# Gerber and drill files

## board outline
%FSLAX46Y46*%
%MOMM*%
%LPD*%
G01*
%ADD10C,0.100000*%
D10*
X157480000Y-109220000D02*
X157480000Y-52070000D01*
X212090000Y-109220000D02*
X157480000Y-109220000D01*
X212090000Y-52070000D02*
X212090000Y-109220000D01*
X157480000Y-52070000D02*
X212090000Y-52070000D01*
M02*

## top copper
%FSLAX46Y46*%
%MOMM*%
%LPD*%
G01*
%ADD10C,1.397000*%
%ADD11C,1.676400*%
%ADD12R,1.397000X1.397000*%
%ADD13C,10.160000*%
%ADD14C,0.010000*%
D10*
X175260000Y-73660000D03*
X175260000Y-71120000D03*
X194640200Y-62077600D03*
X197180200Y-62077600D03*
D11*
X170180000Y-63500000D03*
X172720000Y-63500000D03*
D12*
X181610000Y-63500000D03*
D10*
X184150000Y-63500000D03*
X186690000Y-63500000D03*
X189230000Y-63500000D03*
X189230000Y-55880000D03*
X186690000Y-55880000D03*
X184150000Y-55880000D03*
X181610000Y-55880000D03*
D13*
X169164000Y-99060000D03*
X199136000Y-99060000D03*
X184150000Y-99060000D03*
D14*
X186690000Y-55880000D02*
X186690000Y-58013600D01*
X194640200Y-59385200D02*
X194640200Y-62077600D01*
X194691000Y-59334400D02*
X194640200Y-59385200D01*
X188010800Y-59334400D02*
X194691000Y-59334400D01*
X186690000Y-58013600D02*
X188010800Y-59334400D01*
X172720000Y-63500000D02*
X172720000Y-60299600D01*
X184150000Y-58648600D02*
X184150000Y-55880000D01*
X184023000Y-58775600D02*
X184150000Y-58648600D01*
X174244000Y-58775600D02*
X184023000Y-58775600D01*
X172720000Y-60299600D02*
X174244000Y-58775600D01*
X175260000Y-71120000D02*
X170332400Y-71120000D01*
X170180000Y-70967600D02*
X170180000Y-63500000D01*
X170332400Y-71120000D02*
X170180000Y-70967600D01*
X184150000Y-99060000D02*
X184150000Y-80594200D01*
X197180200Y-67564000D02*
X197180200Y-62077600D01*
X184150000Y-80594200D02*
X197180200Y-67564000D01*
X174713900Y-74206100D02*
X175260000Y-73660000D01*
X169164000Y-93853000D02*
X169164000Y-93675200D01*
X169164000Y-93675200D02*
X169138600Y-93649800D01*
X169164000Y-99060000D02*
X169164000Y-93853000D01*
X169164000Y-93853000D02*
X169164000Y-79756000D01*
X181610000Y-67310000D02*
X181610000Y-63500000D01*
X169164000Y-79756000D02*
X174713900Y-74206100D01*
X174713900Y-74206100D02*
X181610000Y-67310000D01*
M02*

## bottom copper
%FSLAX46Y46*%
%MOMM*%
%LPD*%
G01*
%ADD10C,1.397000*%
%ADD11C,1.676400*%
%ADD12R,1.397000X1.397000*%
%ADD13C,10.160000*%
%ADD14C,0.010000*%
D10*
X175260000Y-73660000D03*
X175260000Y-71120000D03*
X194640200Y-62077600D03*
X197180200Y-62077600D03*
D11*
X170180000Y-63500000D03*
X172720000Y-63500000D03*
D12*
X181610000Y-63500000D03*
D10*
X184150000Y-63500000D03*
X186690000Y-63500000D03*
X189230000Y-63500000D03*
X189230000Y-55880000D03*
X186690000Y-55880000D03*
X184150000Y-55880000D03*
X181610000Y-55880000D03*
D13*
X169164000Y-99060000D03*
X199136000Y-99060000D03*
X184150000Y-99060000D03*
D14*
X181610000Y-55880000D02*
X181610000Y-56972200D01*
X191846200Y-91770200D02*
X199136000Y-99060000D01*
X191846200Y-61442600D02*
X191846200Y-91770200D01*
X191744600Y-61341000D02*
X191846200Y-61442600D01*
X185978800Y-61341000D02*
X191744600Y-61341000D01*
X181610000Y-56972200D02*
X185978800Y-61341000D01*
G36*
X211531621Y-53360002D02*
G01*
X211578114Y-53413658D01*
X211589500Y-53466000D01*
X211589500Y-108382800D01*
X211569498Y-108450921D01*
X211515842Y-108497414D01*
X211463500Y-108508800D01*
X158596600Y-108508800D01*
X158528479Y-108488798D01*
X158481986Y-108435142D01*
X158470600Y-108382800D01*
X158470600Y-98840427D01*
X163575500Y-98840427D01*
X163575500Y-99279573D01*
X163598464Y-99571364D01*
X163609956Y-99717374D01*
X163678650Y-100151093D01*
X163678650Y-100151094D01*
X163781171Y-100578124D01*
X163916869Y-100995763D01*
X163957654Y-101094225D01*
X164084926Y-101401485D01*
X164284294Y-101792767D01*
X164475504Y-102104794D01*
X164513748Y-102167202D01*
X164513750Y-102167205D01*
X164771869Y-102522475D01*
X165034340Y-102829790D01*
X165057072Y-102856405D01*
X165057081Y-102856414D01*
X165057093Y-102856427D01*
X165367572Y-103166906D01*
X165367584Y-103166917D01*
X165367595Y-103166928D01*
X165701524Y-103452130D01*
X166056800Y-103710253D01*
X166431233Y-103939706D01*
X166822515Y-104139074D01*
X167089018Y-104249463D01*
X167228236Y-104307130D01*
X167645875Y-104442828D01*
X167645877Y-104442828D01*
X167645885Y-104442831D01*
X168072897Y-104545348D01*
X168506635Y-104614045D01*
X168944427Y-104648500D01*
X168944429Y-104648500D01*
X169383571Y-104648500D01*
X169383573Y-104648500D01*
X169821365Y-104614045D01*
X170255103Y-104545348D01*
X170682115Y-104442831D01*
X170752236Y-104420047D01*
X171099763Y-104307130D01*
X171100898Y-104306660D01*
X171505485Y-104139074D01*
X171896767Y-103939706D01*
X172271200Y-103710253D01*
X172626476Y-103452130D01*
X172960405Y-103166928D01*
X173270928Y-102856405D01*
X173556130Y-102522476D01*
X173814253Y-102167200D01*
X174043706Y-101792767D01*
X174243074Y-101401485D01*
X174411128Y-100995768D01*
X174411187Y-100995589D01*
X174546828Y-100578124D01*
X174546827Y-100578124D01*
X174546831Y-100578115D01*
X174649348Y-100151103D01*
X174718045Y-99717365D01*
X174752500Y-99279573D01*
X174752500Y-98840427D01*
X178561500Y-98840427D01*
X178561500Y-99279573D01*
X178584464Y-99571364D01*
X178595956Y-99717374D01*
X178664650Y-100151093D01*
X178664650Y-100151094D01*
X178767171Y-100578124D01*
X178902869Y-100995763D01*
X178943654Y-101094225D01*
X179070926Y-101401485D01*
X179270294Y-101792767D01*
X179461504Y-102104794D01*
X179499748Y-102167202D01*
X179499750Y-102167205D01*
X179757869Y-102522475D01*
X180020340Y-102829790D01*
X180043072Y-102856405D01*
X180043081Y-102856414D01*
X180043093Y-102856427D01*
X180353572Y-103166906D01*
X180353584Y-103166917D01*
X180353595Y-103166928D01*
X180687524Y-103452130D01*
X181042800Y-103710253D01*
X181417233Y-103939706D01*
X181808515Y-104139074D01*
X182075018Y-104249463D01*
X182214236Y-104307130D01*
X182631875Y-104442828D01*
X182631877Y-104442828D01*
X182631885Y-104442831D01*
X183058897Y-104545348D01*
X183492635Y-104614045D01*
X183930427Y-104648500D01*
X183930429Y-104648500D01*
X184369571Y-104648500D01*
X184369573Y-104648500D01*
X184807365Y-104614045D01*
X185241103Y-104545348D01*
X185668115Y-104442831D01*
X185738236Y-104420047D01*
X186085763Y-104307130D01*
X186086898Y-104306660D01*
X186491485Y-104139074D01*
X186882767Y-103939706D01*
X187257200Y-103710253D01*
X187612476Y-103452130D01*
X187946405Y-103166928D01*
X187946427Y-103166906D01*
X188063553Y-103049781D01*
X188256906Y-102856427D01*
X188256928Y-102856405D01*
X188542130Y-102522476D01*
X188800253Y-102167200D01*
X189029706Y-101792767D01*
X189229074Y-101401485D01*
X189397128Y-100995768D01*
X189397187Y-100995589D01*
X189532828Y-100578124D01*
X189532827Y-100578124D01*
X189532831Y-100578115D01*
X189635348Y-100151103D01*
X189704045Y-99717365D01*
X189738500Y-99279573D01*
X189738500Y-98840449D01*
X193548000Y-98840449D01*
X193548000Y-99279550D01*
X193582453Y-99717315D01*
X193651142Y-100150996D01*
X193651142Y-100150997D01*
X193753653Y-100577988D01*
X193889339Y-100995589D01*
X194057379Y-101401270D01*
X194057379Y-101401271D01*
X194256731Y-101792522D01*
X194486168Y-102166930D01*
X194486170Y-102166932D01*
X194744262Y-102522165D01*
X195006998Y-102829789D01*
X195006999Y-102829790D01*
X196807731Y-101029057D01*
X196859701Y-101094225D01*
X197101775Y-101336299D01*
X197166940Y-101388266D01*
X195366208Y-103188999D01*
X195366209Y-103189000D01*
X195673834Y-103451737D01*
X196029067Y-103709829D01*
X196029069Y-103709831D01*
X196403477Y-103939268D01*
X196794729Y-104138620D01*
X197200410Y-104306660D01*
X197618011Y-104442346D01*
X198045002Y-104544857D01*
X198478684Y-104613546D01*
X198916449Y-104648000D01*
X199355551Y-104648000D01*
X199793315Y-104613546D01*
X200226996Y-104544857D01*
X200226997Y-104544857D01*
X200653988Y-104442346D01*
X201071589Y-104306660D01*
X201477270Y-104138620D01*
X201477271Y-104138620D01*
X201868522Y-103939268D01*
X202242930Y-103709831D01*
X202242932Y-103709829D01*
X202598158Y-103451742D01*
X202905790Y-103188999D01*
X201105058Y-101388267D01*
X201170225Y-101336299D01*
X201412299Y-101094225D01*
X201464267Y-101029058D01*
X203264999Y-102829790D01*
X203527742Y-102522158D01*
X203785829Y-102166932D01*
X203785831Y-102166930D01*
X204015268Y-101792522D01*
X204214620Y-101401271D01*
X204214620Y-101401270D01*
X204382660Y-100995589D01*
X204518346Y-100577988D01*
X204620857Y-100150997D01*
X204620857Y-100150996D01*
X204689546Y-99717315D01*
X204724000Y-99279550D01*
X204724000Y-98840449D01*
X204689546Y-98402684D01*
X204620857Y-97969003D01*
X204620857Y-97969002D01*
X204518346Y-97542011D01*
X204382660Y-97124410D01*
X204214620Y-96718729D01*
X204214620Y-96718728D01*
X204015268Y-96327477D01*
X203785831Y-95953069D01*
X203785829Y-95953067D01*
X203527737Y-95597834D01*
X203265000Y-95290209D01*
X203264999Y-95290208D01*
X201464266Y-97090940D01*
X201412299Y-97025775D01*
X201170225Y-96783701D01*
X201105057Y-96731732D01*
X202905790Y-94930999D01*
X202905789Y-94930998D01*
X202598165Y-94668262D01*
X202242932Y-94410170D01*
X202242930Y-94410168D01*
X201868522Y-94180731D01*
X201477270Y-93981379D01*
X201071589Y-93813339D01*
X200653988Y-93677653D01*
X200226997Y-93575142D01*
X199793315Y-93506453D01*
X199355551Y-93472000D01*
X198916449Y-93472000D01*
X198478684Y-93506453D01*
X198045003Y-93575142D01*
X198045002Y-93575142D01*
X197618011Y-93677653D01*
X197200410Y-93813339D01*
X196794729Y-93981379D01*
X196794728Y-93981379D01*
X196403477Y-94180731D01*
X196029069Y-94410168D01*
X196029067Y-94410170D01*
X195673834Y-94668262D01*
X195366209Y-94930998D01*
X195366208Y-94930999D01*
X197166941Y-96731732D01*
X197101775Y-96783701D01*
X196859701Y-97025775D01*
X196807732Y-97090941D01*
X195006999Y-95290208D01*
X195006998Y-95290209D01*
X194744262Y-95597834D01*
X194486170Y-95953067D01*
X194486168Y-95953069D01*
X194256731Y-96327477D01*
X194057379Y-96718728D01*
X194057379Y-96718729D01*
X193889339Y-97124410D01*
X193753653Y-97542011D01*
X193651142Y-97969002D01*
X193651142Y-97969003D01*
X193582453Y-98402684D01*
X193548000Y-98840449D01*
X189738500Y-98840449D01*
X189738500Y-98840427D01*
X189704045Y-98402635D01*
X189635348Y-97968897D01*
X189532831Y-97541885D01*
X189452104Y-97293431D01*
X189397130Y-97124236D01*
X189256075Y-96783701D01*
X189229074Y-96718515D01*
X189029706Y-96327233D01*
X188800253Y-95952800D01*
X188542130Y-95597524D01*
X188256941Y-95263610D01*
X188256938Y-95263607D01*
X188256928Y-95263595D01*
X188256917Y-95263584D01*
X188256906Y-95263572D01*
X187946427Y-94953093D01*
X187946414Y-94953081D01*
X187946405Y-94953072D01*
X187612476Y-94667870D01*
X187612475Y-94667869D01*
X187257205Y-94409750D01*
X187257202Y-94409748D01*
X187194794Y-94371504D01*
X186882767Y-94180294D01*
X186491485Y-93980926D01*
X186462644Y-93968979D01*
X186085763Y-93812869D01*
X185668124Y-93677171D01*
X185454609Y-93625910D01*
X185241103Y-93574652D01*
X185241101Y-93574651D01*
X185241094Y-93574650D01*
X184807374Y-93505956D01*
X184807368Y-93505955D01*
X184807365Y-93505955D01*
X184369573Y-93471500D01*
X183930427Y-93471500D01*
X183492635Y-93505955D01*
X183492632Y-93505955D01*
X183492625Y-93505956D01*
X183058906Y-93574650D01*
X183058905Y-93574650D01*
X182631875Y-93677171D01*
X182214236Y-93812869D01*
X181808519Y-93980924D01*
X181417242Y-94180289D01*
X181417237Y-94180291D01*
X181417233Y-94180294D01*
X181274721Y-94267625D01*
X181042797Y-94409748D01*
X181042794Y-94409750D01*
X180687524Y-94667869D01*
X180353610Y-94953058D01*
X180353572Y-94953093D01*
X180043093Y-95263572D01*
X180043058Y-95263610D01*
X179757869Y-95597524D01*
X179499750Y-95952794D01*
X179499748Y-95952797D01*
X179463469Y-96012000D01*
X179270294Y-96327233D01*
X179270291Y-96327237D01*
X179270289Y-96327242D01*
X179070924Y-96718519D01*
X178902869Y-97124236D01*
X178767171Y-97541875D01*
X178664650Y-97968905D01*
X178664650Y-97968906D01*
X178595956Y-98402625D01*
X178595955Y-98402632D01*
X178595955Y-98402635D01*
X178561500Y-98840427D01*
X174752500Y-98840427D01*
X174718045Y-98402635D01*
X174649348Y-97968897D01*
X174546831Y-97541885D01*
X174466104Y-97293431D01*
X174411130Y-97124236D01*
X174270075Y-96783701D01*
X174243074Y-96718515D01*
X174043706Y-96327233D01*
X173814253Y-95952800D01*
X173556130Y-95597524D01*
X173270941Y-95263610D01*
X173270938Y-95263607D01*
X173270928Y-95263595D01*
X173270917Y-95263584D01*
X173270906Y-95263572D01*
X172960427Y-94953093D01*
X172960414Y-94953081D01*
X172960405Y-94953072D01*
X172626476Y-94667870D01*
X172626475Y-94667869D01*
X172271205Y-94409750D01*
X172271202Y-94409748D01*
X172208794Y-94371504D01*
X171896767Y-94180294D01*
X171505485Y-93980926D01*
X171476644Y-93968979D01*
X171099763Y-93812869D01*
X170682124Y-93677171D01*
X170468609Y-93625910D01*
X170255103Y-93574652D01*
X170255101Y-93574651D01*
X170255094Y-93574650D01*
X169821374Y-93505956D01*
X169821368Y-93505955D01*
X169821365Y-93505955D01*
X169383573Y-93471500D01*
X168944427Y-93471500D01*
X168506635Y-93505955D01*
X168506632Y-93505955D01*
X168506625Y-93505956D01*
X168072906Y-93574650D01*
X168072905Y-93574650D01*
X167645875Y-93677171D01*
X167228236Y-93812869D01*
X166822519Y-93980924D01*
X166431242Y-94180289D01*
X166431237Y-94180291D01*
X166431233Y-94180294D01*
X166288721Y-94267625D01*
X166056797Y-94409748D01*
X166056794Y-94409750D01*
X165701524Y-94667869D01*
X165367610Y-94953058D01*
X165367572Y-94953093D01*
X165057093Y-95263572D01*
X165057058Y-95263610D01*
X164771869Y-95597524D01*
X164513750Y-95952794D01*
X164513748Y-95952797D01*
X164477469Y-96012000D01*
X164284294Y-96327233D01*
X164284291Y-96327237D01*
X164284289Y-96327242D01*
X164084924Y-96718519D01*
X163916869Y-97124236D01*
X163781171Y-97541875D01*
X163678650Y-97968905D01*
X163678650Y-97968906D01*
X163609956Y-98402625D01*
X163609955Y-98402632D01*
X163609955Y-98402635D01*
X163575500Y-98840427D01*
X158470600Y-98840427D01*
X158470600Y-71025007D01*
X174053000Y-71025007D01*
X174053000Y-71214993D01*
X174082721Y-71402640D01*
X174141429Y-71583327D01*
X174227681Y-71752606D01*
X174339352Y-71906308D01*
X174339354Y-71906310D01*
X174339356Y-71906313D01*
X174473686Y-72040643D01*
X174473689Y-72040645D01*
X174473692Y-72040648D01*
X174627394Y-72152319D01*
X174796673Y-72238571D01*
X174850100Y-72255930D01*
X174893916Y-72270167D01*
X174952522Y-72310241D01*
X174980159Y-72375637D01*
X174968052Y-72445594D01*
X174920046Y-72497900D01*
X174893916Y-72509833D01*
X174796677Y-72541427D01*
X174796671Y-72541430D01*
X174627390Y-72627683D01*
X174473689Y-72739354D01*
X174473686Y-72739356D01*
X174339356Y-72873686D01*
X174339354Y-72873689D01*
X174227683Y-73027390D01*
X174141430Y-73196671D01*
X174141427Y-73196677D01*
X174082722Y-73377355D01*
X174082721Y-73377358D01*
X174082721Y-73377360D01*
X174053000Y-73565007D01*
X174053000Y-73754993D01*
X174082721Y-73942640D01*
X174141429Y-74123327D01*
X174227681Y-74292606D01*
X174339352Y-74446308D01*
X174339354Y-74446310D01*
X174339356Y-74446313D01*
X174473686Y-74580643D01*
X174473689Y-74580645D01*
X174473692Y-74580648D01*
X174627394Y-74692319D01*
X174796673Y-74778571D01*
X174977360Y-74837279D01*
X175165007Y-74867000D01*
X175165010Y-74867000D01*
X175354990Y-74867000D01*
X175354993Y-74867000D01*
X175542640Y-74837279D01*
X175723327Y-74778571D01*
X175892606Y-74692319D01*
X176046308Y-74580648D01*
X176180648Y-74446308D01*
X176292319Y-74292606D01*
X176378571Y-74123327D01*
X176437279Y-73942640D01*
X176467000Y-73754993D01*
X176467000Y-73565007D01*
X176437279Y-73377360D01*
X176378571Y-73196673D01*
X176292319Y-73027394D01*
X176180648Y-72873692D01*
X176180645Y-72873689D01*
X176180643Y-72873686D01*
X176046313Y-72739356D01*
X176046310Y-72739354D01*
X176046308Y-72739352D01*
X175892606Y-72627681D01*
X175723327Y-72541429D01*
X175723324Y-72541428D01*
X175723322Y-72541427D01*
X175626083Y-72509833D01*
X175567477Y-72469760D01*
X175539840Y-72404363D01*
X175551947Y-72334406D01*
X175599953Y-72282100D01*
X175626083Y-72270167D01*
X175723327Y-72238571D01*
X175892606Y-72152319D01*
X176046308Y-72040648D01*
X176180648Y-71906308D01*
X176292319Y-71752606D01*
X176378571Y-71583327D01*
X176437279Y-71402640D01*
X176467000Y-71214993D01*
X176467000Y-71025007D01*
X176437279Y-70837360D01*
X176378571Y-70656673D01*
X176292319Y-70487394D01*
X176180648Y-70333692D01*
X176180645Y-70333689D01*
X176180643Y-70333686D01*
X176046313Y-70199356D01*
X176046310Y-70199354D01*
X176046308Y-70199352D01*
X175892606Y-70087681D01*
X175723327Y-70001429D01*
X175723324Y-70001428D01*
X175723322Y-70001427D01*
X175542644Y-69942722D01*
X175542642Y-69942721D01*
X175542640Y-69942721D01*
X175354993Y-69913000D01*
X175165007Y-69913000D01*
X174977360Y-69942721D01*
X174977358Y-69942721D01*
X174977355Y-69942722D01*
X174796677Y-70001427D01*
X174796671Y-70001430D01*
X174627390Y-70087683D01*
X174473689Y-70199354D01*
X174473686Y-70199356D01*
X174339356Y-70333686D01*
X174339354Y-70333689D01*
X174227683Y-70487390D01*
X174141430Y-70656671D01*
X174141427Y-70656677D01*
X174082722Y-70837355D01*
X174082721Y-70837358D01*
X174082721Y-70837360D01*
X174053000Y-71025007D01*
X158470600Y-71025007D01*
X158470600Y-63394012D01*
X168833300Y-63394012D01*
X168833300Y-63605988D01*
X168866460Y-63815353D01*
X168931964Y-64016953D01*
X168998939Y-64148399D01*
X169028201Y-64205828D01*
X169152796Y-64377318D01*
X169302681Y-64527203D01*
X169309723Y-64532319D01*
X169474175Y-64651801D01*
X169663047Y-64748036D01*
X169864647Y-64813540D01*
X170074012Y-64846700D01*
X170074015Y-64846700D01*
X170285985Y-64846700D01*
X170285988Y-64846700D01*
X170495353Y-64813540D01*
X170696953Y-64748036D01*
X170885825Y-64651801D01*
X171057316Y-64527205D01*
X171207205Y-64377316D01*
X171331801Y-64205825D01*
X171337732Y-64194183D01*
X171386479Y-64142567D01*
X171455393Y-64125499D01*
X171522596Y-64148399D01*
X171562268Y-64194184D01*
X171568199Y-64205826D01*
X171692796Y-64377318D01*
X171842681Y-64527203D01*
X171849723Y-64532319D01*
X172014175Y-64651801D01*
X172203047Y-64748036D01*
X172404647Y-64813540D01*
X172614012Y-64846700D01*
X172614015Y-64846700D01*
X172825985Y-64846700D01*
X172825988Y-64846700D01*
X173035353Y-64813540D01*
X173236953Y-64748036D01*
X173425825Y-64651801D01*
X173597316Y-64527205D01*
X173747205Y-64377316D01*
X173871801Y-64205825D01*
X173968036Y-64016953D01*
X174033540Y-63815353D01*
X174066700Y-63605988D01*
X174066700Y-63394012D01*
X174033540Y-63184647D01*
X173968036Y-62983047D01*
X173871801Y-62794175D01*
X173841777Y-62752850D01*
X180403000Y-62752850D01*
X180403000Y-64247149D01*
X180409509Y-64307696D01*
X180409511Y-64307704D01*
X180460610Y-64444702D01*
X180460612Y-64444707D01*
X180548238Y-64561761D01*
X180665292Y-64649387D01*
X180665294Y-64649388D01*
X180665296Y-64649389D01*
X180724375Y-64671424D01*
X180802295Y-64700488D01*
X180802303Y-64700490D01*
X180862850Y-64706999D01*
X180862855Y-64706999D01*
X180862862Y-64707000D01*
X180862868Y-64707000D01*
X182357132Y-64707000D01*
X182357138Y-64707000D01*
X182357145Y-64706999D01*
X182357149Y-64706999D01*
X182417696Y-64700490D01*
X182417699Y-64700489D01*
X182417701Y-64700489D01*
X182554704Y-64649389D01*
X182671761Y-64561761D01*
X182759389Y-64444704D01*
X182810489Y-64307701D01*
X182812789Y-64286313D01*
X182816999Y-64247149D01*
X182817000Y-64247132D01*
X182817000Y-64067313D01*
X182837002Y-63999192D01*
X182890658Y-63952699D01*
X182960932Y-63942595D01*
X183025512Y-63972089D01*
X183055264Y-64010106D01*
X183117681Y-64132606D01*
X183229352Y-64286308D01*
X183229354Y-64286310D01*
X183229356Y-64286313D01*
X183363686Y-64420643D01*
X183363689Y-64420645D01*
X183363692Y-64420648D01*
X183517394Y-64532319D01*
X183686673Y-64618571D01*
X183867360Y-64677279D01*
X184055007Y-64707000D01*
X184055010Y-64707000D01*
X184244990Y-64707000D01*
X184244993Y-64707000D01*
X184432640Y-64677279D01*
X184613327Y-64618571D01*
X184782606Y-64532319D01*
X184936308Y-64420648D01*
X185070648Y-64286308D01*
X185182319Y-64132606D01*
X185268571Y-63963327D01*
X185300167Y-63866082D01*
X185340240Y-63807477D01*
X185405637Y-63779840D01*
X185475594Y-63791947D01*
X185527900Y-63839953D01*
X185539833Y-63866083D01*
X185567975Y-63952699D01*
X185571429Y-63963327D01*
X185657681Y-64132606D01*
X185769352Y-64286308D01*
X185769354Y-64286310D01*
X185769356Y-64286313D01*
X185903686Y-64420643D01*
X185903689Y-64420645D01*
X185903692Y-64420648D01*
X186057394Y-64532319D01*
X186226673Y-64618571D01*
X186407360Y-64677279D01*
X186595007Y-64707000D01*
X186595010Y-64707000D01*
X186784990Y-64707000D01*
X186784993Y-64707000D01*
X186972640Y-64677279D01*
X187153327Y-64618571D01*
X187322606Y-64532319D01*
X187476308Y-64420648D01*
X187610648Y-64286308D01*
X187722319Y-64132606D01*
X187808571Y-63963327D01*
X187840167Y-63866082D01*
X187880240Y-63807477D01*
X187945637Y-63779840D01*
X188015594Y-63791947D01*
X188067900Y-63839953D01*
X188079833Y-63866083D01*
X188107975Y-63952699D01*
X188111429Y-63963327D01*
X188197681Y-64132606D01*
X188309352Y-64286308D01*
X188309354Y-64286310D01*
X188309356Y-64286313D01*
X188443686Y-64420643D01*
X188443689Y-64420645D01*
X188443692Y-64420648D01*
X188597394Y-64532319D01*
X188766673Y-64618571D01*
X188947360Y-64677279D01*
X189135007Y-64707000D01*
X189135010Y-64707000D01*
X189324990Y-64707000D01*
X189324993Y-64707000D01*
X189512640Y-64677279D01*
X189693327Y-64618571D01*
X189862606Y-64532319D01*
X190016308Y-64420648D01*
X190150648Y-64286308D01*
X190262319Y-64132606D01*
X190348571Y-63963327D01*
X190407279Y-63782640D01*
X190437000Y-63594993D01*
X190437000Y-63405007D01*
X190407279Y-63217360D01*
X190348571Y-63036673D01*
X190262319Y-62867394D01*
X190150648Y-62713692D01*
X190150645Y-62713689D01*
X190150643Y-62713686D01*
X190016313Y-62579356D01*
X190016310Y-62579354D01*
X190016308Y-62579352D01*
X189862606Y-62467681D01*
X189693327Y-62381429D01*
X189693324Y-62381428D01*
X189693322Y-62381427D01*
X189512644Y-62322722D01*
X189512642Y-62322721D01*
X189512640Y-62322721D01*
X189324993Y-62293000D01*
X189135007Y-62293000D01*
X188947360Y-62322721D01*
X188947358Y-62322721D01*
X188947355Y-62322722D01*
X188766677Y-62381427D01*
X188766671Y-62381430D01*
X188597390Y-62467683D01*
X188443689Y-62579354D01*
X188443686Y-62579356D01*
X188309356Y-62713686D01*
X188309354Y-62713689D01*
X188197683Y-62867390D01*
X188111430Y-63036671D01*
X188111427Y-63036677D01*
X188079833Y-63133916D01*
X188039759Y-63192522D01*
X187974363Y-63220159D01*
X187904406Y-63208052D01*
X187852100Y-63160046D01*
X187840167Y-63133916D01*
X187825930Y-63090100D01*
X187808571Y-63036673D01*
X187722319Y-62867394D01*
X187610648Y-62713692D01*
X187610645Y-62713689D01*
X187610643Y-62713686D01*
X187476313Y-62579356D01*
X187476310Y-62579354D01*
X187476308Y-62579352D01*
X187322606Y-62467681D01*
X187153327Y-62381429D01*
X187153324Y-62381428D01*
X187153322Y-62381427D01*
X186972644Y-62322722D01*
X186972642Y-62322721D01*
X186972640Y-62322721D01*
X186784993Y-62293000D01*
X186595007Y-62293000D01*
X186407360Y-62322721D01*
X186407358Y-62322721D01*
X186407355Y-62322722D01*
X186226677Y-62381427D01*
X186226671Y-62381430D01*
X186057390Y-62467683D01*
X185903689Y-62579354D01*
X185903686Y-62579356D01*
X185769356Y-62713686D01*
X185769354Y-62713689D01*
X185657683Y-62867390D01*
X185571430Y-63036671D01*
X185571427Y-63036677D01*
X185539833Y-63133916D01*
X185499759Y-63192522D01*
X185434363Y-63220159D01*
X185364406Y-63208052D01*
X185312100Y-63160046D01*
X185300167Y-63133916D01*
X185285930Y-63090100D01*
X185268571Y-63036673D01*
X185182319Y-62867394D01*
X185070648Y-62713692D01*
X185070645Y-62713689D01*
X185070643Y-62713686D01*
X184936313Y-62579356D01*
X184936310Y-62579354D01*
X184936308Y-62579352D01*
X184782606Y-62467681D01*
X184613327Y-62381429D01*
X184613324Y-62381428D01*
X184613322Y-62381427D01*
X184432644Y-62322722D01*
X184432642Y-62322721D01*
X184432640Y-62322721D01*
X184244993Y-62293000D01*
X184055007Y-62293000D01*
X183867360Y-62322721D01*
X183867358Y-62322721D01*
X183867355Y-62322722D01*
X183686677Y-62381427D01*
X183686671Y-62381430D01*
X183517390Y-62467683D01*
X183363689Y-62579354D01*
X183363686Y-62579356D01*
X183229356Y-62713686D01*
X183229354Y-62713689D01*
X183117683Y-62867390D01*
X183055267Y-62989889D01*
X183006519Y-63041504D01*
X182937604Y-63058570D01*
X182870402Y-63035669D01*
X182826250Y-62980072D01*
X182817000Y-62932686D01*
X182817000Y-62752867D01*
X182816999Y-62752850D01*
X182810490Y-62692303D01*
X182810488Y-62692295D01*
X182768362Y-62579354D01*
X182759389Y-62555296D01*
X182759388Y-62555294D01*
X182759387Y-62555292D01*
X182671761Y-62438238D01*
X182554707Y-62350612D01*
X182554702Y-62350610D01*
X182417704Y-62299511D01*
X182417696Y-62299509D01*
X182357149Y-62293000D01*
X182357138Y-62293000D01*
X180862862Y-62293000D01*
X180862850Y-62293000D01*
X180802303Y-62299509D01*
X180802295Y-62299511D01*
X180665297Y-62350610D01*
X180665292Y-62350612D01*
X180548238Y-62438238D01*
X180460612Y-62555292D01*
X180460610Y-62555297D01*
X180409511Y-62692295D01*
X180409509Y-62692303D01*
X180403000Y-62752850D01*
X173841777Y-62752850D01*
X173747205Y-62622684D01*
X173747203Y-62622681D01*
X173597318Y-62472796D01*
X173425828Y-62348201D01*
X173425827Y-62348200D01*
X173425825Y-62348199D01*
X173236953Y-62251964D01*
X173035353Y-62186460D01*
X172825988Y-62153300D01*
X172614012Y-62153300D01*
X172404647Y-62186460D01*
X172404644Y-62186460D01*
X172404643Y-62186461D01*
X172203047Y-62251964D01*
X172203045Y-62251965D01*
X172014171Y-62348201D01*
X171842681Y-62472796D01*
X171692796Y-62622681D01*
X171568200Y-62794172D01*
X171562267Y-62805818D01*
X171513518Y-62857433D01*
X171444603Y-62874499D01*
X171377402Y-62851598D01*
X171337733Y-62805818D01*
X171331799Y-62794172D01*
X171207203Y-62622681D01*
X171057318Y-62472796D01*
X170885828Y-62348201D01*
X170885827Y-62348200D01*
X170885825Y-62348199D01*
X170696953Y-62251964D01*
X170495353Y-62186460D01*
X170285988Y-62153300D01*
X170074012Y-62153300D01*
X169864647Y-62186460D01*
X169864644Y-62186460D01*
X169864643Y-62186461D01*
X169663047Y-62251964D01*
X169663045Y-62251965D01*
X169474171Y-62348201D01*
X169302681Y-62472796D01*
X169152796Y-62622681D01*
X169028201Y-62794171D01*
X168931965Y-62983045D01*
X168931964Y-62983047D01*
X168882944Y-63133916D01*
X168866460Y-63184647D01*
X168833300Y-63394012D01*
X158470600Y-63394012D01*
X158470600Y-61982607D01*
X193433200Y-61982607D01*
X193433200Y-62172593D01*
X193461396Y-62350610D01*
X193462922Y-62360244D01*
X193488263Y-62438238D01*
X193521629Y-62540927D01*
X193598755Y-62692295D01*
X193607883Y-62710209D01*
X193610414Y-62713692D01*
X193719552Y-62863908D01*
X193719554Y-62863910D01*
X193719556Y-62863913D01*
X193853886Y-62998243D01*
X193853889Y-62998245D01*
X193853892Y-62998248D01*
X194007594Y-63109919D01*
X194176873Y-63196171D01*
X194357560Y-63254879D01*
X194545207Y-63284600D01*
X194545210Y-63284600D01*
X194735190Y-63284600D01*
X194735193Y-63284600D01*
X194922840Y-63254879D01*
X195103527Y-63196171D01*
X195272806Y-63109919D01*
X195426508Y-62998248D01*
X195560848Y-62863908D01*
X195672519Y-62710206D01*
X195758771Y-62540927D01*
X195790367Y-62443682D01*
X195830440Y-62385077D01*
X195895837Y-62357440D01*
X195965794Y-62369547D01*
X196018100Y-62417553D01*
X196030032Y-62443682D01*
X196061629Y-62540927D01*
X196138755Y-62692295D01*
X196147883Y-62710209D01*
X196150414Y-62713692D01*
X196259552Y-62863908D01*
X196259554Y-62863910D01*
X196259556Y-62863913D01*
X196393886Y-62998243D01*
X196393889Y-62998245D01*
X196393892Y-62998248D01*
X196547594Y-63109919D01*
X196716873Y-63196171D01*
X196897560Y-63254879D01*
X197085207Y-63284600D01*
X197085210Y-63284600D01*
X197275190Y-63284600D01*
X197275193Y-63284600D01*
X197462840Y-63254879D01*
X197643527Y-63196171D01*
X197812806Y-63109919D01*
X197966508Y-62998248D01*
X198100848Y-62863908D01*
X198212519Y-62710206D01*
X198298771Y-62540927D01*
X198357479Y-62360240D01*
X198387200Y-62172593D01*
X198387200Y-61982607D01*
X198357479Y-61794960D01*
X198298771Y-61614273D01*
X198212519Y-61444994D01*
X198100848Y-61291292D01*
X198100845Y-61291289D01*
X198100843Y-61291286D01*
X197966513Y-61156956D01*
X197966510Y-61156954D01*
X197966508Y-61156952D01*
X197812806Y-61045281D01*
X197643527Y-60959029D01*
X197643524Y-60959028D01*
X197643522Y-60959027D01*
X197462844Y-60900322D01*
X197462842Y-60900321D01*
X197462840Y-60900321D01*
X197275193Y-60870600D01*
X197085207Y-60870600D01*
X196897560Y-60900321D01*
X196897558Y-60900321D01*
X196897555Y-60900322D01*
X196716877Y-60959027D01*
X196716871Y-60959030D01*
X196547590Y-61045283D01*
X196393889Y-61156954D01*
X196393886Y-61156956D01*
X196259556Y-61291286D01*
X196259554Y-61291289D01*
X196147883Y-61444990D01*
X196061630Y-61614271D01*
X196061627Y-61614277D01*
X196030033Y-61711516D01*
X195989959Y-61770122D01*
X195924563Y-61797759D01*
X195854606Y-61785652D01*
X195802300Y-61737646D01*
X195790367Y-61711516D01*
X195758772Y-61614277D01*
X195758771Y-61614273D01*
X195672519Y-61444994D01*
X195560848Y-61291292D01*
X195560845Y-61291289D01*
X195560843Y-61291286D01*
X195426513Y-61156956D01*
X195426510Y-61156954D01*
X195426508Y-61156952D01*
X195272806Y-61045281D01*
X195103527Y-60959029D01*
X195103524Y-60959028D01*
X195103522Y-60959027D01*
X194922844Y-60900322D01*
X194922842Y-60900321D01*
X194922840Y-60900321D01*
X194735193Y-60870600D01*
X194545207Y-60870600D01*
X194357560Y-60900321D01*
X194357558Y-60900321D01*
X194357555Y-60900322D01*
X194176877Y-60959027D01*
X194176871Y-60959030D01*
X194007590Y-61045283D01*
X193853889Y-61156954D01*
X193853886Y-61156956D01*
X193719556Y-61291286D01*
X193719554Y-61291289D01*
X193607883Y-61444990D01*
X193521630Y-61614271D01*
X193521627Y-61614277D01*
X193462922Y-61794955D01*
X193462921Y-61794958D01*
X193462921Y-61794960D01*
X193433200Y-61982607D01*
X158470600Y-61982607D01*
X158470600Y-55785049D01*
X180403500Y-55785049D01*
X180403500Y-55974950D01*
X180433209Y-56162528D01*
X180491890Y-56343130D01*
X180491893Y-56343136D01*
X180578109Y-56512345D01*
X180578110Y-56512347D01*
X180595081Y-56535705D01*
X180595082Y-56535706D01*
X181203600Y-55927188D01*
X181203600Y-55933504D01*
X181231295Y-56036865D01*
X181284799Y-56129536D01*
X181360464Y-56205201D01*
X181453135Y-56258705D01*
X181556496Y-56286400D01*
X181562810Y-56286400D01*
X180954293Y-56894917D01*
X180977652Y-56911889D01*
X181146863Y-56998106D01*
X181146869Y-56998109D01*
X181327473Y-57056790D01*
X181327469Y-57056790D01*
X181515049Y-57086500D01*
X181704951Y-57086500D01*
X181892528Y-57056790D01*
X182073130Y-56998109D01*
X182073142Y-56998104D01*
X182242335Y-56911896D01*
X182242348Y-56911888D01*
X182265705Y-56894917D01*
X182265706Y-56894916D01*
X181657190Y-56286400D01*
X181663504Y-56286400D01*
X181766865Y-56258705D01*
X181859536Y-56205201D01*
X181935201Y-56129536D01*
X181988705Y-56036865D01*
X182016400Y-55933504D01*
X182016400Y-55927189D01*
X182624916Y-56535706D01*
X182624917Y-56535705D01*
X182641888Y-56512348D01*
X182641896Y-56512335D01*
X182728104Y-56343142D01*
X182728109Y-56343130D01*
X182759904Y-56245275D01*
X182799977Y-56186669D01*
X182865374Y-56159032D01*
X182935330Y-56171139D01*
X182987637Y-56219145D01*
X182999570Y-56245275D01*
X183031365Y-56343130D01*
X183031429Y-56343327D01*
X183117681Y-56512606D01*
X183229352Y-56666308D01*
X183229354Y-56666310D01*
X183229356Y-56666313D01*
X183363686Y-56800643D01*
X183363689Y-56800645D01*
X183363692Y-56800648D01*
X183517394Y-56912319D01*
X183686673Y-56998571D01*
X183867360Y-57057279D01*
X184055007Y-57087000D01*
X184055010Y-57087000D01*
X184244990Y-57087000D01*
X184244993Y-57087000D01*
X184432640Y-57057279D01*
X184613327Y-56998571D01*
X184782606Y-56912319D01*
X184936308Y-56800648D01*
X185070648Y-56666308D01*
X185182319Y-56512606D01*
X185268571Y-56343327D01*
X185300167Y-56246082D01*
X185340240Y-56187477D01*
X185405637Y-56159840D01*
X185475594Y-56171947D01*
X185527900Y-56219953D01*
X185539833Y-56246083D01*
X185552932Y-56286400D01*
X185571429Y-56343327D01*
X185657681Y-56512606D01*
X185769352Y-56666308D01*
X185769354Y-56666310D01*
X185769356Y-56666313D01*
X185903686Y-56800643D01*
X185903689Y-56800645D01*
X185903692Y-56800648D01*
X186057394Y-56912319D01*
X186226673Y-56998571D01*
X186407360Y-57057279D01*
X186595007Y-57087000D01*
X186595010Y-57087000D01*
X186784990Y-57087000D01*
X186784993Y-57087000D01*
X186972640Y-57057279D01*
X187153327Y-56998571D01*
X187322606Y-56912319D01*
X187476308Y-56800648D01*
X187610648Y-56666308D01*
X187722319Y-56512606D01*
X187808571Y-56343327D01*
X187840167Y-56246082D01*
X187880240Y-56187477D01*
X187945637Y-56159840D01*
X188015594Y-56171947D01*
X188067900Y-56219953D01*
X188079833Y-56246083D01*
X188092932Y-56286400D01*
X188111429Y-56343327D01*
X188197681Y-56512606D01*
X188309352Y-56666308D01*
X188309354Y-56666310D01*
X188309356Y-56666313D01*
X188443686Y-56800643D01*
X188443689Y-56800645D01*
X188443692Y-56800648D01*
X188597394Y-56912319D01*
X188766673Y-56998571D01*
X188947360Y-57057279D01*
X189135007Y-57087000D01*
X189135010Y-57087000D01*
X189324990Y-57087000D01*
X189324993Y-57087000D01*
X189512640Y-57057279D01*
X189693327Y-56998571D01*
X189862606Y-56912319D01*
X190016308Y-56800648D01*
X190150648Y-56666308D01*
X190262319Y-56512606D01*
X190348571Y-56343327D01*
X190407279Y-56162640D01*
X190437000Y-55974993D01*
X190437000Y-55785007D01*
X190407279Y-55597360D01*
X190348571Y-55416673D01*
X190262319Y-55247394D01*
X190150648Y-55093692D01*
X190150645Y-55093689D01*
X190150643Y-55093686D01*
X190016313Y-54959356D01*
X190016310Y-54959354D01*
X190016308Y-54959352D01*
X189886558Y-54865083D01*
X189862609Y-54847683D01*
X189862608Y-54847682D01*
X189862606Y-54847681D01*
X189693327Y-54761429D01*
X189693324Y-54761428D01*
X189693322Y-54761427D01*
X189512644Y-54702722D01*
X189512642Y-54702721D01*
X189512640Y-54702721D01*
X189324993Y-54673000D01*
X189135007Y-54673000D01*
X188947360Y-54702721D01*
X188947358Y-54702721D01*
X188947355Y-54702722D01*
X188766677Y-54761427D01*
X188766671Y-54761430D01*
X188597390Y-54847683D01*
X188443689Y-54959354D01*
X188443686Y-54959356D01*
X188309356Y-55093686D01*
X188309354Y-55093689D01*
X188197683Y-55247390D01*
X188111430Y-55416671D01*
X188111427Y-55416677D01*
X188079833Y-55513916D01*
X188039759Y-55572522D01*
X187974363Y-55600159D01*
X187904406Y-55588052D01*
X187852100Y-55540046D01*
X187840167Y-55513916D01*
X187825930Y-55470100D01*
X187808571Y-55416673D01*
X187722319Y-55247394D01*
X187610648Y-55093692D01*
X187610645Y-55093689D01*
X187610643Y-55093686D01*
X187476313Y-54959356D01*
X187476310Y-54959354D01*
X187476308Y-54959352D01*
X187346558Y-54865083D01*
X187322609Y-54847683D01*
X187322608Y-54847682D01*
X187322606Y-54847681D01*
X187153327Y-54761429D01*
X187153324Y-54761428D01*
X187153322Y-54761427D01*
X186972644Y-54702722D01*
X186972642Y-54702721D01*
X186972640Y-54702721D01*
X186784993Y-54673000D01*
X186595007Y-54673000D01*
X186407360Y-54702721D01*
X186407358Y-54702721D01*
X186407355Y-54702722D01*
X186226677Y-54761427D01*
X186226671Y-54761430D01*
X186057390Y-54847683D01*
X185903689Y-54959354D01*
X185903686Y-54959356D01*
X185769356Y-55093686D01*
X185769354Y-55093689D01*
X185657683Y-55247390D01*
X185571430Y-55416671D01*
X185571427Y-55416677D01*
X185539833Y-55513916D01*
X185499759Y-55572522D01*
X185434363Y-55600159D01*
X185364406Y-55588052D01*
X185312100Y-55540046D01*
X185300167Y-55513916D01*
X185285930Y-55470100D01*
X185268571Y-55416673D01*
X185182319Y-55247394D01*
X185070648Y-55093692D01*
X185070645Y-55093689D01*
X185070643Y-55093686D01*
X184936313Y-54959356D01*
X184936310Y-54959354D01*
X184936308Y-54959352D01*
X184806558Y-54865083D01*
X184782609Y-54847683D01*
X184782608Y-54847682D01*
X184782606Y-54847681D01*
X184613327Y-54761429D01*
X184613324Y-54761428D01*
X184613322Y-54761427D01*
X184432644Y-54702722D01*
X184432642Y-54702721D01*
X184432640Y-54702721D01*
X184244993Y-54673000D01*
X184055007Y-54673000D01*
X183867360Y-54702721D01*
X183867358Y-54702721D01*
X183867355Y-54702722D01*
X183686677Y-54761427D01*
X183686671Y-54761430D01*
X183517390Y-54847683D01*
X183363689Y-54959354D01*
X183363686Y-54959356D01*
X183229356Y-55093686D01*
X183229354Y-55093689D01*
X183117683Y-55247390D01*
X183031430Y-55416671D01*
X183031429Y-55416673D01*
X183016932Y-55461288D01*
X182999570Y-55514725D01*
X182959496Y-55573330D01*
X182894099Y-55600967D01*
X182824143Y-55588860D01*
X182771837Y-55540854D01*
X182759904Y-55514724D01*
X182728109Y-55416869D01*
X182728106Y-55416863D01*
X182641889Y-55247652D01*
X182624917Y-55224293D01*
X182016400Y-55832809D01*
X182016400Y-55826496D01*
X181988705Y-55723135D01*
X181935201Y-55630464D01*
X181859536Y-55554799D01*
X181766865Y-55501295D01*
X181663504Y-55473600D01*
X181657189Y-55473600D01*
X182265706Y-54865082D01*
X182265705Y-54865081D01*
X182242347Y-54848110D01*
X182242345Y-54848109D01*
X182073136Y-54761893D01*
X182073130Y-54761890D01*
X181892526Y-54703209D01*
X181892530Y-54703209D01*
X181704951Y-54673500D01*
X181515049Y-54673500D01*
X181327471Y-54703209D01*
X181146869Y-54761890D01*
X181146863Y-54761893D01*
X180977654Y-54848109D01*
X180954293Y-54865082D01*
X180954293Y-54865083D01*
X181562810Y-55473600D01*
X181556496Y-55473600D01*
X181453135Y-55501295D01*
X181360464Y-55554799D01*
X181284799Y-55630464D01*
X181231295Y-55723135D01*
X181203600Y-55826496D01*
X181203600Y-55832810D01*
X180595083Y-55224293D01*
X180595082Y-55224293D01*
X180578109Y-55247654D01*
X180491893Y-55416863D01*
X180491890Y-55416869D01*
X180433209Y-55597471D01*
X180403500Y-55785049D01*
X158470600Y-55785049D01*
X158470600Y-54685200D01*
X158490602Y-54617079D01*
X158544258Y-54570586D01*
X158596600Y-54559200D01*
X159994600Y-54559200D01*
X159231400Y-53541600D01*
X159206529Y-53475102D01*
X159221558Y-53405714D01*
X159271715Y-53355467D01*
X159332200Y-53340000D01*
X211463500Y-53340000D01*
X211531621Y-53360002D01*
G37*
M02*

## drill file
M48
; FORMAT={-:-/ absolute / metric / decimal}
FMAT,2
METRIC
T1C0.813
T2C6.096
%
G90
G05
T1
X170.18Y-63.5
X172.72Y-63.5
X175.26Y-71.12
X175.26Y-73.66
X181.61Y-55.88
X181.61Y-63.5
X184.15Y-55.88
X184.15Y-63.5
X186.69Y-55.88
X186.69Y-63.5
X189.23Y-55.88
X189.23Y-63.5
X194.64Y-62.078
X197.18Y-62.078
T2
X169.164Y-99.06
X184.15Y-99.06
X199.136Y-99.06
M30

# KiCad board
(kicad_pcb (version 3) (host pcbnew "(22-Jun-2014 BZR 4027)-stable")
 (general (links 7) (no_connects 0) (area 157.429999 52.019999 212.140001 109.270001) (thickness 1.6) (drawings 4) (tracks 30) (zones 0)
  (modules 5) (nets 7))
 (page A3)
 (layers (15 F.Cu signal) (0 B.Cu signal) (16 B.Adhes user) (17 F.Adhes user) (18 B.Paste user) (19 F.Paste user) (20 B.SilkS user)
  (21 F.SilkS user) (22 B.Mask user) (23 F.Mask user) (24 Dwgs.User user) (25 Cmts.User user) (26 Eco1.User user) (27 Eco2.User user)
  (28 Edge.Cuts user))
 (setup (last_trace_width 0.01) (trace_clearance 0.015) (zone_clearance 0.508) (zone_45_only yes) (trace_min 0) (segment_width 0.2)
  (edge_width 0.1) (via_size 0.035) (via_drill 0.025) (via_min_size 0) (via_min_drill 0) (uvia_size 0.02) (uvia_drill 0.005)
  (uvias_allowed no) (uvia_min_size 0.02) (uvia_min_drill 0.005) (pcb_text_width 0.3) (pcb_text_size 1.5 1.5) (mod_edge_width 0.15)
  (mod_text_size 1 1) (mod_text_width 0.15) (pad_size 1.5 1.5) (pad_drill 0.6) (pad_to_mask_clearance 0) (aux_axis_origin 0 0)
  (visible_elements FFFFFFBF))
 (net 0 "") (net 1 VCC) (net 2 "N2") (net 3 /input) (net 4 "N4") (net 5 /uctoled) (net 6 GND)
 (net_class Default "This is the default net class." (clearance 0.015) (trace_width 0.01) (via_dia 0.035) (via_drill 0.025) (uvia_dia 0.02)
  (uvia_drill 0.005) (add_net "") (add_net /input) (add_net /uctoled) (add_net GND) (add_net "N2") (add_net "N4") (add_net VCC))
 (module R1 (layer F.Cu) (at 175.26 72.39 90) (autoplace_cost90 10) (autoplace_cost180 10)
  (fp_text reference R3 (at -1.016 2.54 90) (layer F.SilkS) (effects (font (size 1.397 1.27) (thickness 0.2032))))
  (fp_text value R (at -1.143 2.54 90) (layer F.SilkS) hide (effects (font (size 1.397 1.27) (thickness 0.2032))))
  (pad 1 thru_hole circle (at -1.27 0 90) (size 1.397 1.397) (drill 0.8128) (layers *.Cu *.Mask F.SilkS) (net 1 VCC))
  (pad 2 thru_hole circle (at 1.27 0 90) (size 1.397 1.397) (drill 0.8128) (layers *.Cu *.Mask F.SilkS) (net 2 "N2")))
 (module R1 (layer F.Cu) (at 195.9102 62.0776) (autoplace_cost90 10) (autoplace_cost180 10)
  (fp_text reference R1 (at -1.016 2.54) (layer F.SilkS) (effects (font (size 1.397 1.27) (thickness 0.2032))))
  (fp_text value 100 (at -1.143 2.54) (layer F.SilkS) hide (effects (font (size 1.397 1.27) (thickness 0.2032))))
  (pad 1 thru_hole circle (at -1.27 0) (size 1.397 1.397) (drill 0.8128) (layers *.Cu *.Mask F.SilkS) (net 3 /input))
  (pad 2 thru_hole circle (at 1.27 0) (size 1.397 1.397) (drill 0.8128) (layers *.Cu *.Mask F.SilkS) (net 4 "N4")))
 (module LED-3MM (layer F.Cu) (at 171.45 63.5)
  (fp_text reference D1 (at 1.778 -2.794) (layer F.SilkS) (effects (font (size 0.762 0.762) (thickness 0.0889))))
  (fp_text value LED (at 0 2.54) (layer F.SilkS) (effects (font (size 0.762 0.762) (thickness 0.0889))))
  (pad 1 thru_hole circle (at -1.27 0) (size 1.6764 1.6764) (drill 0.8128) (layers *.Cu *.Mask F.SilkS) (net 2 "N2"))
  (pad 2 thru_hole circle (at 1.27 0) (size 1.6764 1.6764) (drill 0.8128) (layers *.Cu *.Mask F.SilkS) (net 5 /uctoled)))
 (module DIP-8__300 (layer F.Cu) (at 185.42 59.69)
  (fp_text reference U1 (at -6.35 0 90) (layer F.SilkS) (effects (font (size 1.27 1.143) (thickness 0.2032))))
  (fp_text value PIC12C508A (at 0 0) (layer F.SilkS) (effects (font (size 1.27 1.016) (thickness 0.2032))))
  (pad 1 thru_hole rect (at -3.81 3.81) (size 1.397 1.397) (drill 0.8128) (layers *.Cu *.Mask F.SilkS) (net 1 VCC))
  (pad 2 thru_hole circle (at -1.27 3.81) (size 1.397 1.397) (drill 0.8128) (layers *.Cu *.Mask F.SilkS))
  (pad 3 thru_hole circle (at 1.27 3.81) (size 1.397 1.397) (drill 0.8128) (layers *.Cu *.Mask F.SilkS))
  (pad 4 thru_hole circle (at 3.81 3.81) (size 1.397 1.397) (drill 0.8128) (layers *.Cu *.Mask F.SilkS))
  (pad 5 thru_hole circle (at 3.81 -3.81) (size 1.397 1.397) (drill 0.8128) (layers *.Cu *.Mask F.SilkS))
  (pad 6 thru_hole circle (at 1.27 -3.81) (size 1.397 1.397) (drill 0.8128) (layers *.Cu *.Mask F.SilkS) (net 3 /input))
  (pad 7 thru_hole circle (at -1.27 -3.81) (size 1.397 1.397) (drill 0.8128) (layers *.Cu *.Mask F.SilkS) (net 5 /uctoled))
  (pad 8 thru_hole circle (at -3.81 -3.81) (size 1.397 1.397) (drill 0.8128) (layers *.Cu *.Mask F.SilkS) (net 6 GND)))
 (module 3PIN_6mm (layer F.Cu) (at 184.15 99.06)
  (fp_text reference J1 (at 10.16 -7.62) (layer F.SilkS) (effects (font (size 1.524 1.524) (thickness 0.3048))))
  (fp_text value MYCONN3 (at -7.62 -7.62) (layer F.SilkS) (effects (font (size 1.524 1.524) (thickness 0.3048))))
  (pad 1 thru_hole circle (at -14.986 0) (size 10.16 10.16) (drill 6.096) (layers *.Cu *.Mask F.SilkS) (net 1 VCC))
  (pad 3 thru_hole circle (at 14.986 0) (size 10.16 10.16) (drill 6.096) (layers *.Cu *.Mask F.SilkS) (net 6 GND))
  (pad 2 thru_hole circle (at 0 0) (size 10.16 10.16) (drill 6.096) (layers *.Cu *.Mask F.SilkS) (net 4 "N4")))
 (gr_line (start 157.48 109.22) (end 157.48 52.07) (angle 90) (layer Edge.Cuts) (width 0.1))
 (gr_line (start 212.09 109.22) (end 157.48 109.22) (angle 90) (layer Edge.Cuts) (width 0.1))
 (gr_line (start 212.09 52.07) (end 212.09 109.22) (angle 90) (layer Edge.Cuts) (width 0.1))
 (gr_line (start 157.48 52.07) (end 212.09 52.07) (angle 90) (layer Edge.Cuts) (width 0.1))
 (segment (start 186.69 55.88) (end 186.69 58.0136) (width 0.01) (layer F.Cu) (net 3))
 (segment (start 194.6402 59.3852) (end 194.6402 62.0776) (width 0.01) (layer F.Cu) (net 3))
 (segment (start 194.691 59.3344) (end 194.6402 59.3852) (width 0.01) (layer F.Cu) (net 3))
 (segment (start 188.0108 59.3344) (end 194.691 59.3344) (width 0.01) (layer F.Cu) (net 3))
 (segment (start 186.69 58.0136) (end 188.0108 59.3344) (width 0.01) (layer F.Cu) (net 3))
 (segment (start 172.72 63.5) (end 172.72 60.2996) (width 0.01) (layer F.Cu) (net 5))
 (segment (start 184.15 58.6486) (end 184.15 55.88) (width 0.01) (layer F.Cu) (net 5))
 (segment (start 184.023 58.7756) (end 184.15 58.6486) (width 0.01) (layer F.Cu) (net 5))
 (segment (start 174.244 58.7756) (end 184.023 58.7756) (width 0.01) (layer F.Cu) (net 5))
 (segment (start 172.72 60.2996) (end 174.244 58.7756) (width 0.01) (layer F.Cu) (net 5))
 (segment (start 181.61 55.88) (end 181.61 56.9722) (width 0.01) (layer B.Cu) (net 6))
 (segment (start 191.8462 91.7702) (end 199.136 99.06) (width 0.01) (layer B.Cu) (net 6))
 (segment (start 191.8462 61.4426) (end 191.8462 91.7702) (width 0.01) (layer B.Cu) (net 6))
 (segment (start 191.7446 61.341) (end 191.8462 61.4426) (width 0.01) (layer B.Cu) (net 6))
 (segment (start 185.9788 61.341) (end 191.7446 61.341) (width 0.01) (layer B.Cu) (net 6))
 (segment (start 181.61 56.9722) (end 185.9788 61.341) (width 0.01) (layer B.Cu) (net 6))
 (segment (start 175.26 71.12) (end 170.3324 71.12) (width 0.01) (layer F.Cu) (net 2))
 (segment (start 170.18 70.9676) (end 170.18 63.5) (width 0.01) (layer F.Cu) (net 2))
 (segment (start 170.3324 71.12) (end 170.18 70.9676) (width 0.01) (layer F.Cu) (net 2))
 (segment (start 184.15 99.06) (end 184.15 80.5942) (width 0.01) (layer F.Cu) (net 4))
 (segment (start 197.1802 67.564) (end 197.1802 62.0776) (width 0.01) (layer F.Cu) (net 4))
 (segment (start 184.15 80.5942) (end 197.1802 67.564) (width 0.01) (layer F.Cu) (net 4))
 (segment (start 174.7139 74.2061) (end 175.26 73.66) (width 0.01) (layer F.Cu) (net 1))
 (segment (start 169.164 93.853) (end 169.164 93.6752) (width 0.01) (layer F.Cu) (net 1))
 (segment (start 169.164 93.6752) (end 169.1386 93.6498) (width 0.01) (layer F.Cu) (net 1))
 (segment (start 169.164 99.06) (end 169.164 93.853) (width 0.01) (layer F.Cu) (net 1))
 (segment (start 169.164 93.853) (end 169.164 79.756) (width 0.01) (layer F.Cu) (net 1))
 (segment (start 181.61 67.31) (end 181.61 63.5) (width 0.01) (layer F.Cu) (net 1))
 (segment (start 169.164 79.756) (end 174.7139 74.2061) (width 0.01) (layer F.Cu) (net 1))
 (segment (start 174.7139 74.2061) (end 181.61 67.31) (width 0.01) (layer F.Cu) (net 1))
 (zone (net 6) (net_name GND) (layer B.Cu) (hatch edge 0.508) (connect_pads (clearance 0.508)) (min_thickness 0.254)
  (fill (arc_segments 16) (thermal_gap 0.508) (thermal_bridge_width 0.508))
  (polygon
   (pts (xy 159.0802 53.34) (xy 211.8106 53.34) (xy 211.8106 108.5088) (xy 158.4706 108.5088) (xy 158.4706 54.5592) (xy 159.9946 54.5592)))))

